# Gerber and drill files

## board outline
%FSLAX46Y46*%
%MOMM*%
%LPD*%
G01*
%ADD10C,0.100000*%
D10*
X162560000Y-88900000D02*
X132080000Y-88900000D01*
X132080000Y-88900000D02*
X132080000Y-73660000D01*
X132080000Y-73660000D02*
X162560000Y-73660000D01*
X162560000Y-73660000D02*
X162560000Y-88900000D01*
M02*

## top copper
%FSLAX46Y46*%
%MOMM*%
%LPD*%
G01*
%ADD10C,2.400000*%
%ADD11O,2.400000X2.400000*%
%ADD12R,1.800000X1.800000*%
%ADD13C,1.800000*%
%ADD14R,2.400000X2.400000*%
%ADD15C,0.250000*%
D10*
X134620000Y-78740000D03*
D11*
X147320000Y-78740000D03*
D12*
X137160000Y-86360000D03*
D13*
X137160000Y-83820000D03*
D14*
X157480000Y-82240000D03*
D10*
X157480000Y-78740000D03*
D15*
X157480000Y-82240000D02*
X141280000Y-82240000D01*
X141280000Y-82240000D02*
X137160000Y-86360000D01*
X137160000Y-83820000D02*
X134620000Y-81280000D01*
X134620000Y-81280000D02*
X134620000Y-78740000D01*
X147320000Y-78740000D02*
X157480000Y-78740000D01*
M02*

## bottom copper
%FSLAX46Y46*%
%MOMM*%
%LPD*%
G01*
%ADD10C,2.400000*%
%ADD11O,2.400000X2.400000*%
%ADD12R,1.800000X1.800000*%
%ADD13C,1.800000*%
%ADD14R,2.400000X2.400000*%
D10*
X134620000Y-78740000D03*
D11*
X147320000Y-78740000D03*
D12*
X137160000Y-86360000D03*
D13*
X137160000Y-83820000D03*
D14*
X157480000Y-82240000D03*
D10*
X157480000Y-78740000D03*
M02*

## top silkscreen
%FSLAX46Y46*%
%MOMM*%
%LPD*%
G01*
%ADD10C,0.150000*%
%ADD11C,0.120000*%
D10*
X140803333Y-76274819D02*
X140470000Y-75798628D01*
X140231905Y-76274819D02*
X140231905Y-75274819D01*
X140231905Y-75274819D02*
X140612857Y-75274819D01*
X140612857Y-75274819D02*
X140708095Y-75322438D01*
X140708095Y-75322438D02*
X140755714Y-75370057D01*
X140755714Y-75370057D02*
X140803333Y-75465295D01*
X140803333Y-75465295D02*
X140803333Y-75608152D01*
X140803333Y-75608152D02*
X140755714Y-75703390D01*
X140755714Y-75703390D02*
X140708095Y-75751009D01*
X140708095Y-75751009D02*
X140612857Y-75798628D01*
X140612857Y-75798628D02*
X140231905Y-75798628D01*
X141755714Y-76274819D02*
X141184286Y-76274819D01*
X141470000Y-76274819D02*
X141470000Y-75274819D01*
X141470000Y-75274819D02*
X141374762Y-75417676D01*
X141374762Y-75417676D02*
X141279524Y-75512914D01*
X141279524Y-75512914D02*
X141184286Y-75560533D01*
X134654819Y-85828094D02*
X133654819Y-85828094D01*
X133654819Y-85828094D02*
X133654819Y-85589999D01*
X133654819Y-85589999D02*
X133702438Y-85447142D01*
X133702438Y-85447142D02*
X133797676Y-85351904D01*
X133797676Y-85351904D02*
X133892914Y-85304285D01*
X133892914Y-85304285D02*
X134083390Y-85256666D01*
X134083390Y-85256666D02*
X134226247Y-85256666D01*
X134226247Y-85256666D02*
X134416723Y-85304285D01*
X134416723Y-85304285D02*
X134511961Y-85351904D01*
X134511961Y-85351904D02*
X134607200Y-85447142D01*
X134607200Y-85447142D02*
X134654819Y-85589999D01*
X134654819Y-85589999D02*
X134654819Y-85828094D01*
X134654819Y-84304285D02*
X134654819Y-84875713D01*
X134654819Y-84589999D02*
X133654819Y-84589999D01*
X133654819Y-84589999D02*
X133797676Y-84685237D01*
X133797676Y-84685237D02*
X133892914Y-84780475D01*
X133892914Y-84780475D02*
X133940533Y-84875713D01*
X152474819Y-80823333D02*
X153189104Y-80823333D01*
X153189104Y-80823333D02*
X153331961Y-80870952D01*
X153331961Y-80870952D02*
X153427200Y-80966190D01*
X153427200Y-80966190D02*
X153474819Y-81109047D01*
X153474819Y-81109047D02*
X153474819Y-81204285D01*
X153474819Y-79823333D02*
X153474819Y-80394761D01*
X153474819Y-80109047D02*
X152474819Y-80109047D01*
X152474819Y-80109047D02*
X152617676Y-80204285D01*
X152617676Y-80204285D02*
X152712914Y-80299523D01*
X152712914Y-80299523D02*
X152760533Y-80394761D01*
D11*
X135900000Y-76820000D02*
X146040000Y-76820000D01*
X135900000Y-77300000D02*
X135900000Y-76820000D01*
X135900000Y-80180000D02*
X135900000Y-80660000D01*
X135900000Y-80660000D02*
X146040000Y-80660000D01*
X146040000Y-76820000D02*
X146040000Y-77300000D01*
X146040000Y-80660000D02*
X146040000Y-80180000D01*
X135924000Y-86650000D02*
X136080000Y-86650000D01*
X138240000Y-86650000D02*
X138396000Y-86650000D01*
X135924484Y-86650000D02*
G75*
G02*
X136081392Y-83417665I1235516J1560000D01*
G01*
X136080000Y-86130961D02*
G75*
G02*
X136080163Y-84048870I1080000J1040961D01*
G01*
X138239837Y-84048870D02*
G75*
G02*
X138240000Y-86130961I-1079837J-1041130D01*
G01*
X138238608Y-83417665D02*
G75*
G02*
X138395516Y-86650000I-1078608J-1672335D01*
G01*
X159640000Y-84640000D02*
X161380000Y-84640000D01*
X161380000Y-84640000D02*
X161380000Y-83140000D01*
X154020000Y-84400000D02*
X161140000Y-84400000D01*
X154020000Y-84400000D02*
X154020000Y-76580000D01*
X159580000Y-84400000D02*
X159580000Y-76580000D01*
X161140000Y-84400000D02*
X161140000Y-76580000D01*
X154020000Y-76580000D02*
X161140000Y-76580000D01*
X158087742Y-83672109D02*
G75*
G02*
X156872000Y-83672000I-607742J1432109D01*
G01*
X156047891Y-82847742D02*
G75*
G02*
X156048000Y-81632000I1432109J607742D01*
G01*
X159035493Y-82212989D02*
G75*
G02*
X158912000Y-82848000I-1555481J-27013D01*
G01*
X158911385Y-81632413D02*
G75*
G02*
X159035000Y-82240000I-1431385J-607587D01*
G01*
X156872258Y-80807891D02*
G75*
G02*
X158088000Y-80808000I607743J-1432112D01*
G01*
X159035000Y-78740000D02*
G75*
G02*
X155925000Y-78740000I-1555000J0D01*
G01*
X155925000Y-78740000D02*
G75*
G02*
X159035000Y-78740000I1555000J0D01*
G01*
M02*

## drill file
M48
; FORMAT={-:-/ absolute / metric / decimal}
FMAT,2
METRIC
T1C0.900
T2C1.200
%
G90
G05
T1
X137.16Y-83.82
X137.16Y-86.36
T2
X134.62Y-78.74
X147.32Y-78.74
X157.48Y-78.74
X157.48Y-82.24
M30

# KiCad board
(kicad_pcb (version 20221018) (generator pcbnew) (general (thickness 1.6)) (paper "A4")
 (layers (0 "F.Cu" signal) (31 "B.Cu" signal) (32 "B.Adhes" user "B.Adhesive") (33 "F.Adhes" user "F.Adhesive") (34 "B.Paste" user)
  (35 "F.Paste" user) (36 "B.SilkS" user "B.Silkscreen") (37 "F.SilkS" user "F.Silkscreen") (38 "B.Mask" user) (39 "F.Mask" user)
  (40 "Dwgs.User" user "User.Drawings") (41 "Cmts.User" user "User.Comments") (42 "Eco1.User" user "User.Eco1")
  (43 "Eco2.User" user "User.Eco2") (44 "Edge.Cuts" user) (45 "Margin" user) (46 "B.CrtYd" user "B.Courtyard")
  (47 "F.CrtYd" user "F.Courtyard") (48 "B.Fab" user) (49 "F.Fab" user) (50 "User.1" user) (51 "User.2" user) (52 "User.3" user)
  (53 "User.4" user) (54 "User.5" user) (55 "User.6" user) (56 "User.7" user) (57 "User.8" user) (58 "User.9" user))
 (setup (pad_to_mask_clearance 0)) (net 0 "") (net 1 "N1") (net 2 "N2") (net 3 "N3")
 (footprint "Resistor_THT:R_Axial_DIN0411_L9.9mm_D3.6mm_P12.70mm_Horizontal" (layer "F.Cu") (at 134.62 78.74)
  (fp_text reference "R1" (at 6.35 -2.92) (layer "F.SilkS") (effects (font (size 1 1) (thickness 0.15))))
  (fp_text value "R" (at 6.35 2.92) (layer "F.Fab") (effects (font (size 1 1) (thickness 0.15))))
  (fp_line (start 1.28 -1.92) (end 11.42 -1.92) (stroke (width 0.12) (type solid)) (layer "F.SilkS"))
  (fp_line (start 1.28 -1.44) (end 1.28 -1.92) (stroke (width 0.12) (type solid)) (layer "F.SilkS"))
  (fp_line (start 1.28 1.44) (end 1.28 1.92) (stroke (width 0.12) (type solid)) (layer "F.SilkS"))
  (fp_line (start 1.28 1.92) (end 11.42 1.92) (stroke (width 0.12) (type solid)) (layer "F.SilkS"))
  (fp_line (start 11.42 -1.92) (end 11.42 -1.44) (stroke (width 0.12) (type solid)) (layer "F.SilkS"))
  (fp_line (start 11.42 1.92) (end 11.42 1.44) (stroke (width 0.12) (type solid)) (layer "F.SilkS"))
  (pad "1" thru_hole circle (at 0 0) (size 2.4 2.4) (drill 1.2) (layers "*.Cu" "*.Mask") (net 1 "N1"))
  (pad "2" thru_hole oval (at 12.7 0) (size 2.4 2.4) (drill 1.2) (layers "*.Cu" "*.Mask") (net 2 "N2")))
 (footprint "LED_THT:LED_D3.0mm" (layer "F.Cu") (at 137.16 86.36 90)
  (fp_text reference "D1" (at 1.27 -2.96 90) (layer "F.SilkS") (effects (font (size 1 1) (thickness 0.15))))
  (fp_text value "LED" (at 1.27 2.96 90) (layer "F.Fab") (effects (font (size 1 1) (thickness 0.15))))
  (fp_line (start -0.29 -1.236) (end -0.29 -1.08) (stroke (width 0.12) (type solid)) (layer "F.SilkS"))
  (fp_line (start -0.29 1.08) (end -0.29 1.236) (stroke (width 0.12) (type solid)) (layer "F.SilkS"))
  (fp_arc (start -0.29 -1.235516) (mid 1.366487 -1.987659) (end 2.942335 -1.078608) (stroke (width 0.12) (type solid)) (layer "F.SilkS"))
  (fp_arc (start 0.229039 -1.08) (mid 1.270117 -1.5) (end 2.31113 -1.079837) (stroke (width 0.12) (type solid)) (layer "F.SilkS"))
  (fp_arc (start 2.31113 1.079837) (mid 1.270117 1.5) (end 0.229039 1.08) (stroke (width 0.12) (type solid)) (layer "F.SilkS"))
  (fp_arc (start 2.942335 1.078608) (mid 1.366487 1.987659) (end -0.29 1.235516) (stroke (width 0.12) (type solid)) (layer "F.SilkS"))
  (pad "1" thru_hole rect (at 0 0 90) (size 1.8 1.8) (drill 0.9) (layers "*.Cu" "*.Mask") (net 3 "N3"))
  (pad "2" thru_hole circle (at 2.54 0 90) (size 1.8 1.8) (drill 0.9) (layers "*.Cu" "*.Mask") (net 1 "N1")))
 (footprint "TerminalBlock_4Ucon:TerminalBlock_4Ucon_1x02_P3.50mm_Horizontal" (layer "F.Cu") (at 157.48 82.24 90)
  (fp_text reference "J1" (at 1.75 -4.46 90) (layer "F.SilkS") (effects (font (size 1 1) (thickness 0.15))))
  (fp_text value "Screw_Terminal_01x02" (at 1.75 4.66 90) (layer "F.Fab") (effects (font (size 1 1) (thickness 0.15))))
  (fp_line (start -2.4 2.16) (end -2.4 3.9) (stroke (width 0.12) (type solid)) (layer "F.SilkS"))
  (fp_line (start -2.4 3.9) (end -0.9 3.9) (stroke (width 0.12) (type solid)) (layer "F.SilkS"))
  (fp_line (start -2.16 -3.46) (end -2.16 3.66) (stroke (width 0.12) (type solid)) (layer "F.SilkS"))
  (fp_line (start -2.16 -3.46) (end 5.66 -3.46) (stroke (width 0.12) (type solid)) (layer "F.SilkS"))
  (fp_line (start -2.16 2.1) (end 5.66 2.1) (stroke (width 0.12) (type solid)) (layer "F.SilkS"))
  (fp_line (start -2.16 3.66) (end 5.66 3.66) (stroke (width 0.12) (type solid)) (layer "F.SilkS"))
  (fp_line (start 5.66 -3.46) (end 5.66 3.66) (stroke (width 0.12) (type solid)) (layer "F.SilkS"))
  (fp_arc (start -1.432109 0.607742) (mid -1.555727 -0.00014) (end -1.432 -0.608) (stroke (width 0.12) (type solid)) (layer "F.SilkS"))
  (fp_arc (start -0.607742 -1.432109) (mid 0.00014 -1.555727) (end 0.608 -1.432) (stroke (width 0.12) (type solid)) (layer "F.SilkS"))
  (fp_arc (start 0.027011 1.555493) (mid -0.296984 1.527118) (end -0.608 1.432) (stroke (width 0.12) (type solid)) (layer "F.SilkS"))
  (fp_arc (start 0.607587 1.431385) (mid 0.310017 1.523783) (end 0 1.555) (stroke (width 0.12) (type solid)) (layer "F.SilkS"))
  (fp_arc (start 1.432109 -0.607742) (mid 1.555727 0.00014) (end 1.432 0.608) (stroke (width 0.12) (type solid)) (layer "F.SilkS"))
  (fp_circle (center 3.5 0) (end 5.055 0) (stroke (width 0.12) (type solid)) (fill none) (layer "F.SilkS"))
  (pad "1" thru_hole rect (at 0 0 90) (size 2.4 2.4) (drill 1.2) (layers "*.Cu" "*.Mask") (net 3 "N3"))
  (pad "2" thru_hole circle (at 3.5 0 90) (size 2.4 2.4) (drill 1.2) (layers "*.Cu" "*.Mask") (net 2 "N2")))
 (gr_line (start 162.56 88.9) (end 132.08 88.9) (stroke (width 0.1) (type default)) (layer "Edge.Cuts"))
 (gr_line (start 132.08 88.9) (end 132.08 73.66) (stroke (width 0.1) (type default)) (layer "Edge.Cuts"))
 (gr_line (start 132.08 73.66) (end 162.56 73.66) (stroke (width 0.1) (type default)) (layer "Edge.Cuts"))
 (gr_line (start 162.56 73.66) (end 162.56 88.9) (stroke (width 0.1) (type default)) (layer "Edge.Cuts"))
 (segment (start 157.48 82.24) (end 141.28 82.24) (width 0.25) (layer "F.Cu") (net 3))
 (segment (start 141.28 82.24) (end 137.16 86.36) (width 0.25) (layer "F.Cu") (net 3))
 (segment (start 137.16 83.82) (end 134.62 81.28) (width 0.25) (layer "F.Cu") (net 1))
 (segment (start 134.62 81.28) (end 134.62 78.74) (width 0.25) (layer "F.Cu") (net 1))
 (segment (start 147.32 78.74) (end 157.48 78.74) (width 0.25) (layer "F.Cu") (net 2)))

